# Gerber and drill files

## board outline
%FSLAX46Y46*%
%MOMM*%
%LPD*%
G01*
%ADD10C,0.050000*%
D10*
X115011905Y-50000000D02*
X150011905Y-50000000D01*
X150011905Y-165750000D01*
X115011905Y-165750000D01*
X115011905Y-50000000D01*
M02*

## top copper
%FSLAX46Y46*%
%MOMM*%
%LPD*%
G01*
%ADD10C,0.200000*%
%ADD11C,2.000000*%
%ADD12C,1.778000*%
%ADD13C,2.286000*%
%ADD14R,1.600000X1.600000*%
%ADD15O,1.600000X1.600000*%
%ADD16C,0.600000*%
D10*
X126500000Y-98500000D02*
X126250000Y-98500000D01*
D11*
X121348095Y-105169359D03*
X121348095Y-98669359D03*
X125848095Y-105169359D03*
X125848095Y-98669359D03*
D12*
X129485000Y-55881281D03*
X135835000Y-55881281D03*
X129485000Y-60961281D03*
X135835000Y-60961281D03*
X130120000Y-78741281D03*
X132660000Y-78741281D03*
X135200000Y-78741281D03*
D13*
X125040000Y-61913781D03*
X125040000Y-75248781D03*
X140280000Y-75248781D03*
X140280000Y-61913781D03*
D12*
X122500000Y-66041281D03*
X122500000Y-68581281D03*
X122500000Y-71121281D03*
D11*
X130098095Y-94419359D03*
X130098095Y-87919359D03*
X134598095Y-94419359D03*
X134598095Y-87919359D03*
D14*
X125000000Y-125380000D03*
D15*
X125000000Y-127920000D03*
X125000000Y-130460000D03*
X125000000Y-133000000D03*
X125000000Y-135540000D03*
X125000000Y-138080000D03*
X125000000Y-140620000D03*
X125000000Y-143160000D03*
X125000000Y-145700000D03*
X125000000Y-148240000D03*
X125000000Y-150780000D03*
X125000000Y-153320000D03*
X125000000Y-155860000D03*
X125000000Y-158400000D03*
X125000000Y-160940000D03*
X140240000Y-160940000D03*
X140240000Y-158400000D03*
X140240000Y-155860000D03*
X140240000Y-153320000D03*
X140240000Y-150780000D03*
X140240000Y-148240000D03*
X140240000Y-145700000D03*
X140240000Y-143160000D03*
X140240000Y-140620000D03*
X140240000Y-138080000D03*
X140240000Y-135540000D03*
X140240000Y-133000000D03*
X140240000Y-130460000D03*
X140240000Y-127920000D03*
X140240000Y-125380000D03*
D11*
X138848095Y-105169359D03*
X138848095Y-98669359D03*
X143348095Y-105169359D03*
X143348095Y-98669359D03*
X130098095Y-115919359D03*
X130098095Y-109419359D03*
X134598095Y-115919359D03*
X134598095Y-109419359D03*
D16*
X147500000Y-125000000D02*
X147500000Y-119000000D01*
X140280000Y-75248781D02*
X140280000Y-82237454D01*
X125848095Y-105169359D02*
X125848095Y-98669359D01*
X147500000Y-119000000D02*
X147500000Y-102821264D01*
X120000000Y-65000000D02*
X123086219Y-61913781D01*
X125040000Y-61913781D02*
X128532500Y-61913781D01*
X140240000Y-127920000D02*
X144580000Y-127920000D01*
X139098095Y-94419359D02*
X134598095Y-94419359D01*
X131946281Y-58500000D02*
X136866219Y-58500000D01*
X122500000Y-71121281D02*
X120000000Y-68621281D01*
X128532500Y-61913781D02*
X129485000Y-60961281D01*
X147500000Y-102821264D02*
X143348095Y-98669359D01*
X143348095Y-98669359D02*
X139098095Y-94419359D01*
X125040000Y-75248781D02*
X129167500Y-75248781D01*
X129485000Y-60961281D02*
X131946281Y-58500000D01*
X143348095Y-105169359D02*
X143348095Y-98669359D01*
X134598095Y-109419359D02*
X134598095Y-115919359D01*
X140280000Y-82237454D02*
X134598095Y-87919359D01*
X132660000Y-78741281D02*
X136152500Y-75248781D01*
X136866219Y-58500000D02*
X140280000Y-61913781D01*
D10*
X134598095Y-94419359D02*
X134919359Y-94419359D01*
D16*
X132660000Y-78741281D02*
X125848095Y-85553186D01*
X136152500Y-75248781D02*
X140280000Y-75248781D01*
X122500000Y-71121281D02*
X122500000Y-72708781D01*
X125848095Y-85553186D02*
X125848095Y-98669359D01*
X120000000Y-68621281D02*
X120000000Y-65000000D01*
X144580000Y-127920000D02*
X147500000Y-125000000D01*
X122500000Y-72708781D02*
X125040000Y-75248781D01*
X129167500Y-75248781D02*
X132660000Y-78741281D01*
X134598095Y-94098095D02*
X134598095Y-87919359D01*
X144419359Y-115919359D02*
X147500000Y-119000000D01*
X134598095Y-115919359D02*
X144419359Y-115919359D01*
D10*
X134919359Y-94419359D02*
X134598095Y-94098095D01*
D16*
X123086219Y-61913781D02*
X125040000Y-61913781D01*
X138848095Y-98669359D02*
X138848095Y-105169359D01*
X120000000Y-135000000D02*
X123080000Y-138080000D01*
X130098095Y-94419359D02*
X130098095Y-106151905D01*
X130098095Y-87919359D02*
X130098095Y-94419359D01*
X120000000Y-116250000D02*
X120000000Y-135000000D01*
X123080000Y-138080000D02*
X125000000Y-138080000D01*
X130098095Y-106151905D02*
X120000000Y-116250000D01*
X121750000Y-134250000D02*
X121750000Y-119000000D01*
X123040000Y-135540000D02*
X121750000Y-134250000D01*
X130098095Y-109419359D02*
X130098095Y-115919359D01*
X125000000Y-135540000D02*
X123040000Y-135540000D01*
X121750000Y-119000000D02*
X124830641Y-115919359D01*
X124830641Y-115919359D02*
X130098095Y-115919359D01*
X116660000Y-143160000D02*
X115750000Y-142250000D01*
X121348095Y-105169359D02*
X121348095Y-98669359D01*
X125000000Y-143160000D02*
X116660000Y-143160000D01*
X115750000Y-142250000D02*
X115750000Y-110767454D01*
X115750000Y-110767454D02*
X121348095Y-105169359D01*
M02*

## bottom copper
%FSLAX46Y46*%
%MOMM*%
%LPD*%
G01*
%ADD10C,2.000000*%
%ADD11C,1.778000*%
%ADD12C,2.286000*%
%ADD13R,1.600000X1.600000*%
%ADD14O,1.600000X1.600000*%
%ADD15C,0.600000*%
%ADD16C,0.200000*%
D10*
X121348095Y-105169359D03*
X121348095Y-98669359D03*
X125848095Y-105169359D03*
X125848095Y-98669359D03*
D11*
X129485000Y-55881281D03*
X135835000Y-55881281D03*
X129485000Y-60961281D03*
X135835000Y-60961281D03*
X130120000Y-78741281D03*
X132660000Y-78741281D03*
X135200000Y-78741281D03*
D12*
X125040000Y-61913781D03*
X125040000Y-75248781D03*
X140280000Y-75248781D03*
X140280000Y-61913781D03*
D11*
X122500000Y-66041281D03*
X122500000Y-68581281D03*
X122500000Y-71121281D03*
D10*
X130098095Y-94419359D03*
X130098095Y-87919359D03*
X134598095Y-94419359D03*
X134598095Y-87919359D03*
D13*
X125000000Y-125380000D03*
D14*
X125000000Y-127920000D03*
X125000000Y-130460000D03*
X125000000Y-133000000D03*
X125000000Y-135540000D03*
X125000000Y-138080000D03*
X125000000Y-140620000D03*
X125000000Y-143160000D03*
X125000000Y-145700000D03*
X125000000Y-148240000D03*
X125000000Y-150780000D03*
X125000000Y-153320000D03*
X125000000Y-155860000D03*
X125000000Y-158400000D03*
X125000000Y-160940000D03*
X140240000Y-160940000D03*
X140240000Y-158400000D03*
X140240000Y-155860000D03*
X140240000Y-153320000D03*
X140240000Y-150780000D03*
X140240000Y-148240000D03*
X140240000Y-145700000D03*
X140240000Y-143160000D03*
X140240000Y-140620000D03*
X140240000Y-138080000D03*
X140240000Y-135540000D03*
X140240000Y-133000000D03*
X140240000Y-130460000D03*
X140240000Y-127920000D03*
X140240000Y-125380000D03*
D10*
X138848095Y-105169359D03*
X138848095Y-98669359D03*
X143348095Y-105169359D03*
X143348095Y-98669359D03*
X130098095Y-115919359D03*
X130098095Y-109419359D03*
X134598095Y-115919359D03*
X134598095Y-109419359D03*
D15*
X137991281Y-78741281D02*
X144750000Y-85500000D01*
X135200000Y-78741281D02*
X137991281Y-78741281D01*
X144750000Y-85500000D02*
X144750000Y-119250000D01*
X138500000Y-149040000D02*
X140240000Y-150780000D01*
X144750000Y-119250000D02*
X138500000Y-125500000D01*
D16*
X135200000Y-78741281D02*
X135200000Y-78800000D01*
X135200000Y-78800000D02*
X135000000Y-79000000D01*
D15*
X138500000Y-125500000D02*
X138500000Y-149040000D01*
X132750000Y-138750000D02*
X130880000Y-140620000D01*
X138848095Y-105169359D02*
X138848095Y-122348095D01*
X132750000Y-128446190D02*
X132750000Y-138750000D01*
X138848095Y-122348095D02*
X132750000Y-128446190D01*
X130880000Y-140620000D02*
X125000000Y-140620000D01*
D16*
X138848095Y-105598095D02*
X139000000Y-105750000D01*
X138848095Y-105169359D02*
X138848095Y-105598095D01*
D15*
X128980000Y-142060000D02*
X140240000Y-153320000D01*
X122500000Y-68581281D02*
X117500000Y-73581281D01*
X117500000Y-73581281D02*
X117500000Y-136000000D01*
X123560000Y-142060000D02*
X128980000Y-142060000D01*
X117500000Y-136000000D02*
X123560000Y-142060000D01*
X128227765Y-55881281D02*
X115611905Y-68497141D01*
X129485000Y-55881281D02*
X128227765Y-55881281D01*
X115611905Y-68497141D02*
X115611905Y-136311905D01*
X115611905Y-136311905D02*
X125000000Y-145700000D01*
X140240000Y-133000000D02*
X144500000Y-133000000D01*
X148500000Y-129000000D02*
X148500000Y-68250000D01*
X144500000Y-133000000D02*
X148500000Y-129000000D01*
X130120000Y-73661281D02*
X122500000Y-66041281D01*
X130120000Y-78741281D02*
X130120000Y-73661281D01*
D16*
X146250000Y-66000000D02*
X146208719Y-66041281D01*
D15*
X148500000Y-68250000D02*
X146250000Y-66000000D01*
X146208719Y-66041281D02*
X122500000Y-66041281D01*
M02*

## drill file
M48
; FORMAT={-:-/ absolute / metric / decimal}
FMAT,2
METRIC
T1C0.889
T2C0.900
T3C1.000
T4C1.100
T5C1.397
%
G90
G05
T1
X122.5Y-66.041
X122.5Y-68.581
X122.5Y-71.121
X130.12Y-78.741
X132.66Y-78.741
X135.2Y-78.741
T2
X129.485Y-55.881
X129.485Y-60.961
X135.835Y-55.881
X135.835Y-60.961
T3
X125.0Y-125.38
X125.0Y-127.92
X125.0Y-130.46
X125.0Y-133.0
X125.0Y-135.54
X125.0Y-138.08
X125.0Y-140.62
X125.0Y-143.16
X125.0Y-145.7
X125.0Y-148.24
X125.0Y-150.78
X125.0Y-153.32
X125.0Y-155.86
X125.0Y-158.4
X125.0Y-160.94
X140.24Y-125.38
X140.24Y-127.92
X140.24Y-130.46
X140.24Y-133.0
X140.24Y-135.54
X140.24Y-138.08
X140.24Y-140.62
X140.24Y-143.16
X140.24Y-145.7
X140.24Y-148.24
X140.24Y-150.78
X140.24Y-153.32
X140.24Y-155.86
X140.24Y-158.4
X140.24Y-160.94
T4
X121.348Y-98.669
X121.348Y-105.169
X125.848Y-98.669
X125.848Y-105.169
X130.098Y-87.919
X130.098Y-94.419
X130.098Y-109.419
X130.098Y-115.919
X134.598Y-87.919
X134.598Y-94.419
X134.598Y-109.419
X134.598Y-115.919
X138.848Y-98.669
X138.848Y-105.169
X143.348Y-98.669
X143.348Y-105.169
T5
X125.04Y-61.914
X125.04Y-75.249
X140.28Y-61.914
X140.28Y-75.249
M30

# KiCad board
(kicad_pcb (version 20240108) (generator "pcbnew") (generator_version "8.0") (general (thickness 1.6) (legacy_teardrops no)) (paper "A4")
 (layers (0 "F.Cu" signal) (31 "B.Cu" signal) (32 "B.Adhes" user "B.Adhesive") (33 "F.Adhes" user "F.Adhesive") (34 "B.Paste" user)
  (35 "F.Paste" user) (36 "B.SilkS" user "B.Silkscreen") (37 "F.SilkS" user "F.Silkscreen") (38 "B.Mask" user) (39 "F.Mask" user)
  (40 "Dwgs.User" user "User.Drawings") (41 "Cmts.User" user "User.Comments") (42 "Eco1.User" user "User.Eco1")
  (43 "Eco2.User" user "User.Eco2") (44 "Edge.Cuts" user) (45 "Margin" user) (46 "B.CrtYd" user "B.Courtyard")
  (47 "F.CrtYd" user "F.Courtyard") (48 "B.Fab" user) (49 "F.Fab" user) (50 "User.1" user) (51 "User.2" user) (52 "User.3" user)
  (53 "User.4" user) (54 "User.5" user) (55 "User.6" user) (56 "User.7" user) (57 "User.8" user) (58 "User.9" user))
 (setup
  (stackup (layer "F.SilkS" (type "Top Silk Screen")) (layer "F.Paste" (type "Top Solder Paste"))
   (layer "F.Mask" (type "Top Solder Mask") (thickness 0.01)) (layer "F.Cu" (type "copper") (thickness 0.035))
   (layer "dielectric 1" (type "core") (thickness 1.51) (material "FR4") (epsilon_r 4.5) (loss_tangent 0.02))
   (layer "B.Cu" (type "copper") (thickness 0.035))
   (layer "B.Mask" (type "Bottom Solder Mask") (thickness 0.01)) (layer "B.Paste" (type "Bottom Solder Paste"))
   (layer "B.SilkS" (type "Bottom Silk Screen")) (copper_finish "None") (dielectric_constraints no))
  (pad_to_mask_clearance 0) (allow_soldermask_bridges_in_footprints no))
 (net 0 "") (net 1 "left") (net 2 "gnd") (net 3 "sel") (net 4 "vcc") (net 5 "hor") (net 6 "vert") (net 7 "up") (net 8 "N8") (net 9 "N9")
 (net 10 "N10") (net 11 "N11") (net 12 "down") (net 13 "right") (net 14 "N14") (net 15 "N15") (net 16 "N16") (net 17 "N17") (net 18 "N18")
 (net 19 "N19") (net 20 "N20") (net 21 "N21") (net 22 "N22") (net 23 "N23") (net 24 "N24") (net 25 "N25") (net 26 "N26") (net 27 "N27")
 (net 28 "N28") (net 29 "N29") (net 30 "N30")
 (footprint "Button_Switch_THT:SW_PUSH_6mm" (layer "F.Cu") (at 121.348095 105.169359 90)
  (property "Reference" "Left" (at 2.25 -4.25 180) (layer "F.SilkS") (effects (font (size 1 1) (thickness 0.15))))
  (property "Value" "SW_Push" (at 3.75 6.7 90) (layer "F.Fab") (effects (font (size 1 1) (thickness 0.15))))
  (pad "1" thru_hole circle (at 0 0 180) (size 2 2) (drill 1.1) (layers "*.Cu" "*.Mask") (remove_unused_layers no) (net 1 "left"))
  (pad "1" thru_hole circle (at 6.5 0 180) (size 2 2) (drill 1.1) (layers "*.Cu" "*.Mask") (remove_unused_layers no) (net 1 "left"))
  (pad "2" thru_hole circle (at 0 4.5 180) (size 2 2) (drill 1.1) (layers "*.Cu" "*.Mask") (remove_unused_layers no) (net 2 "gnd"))
  (pad "2" thru_hole circle (at 6.5 4.5 180) (size 2 2) (drill 1.1) (layers "*.Cu" "*.Mask") (remove_unused_layers no) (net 2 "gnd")))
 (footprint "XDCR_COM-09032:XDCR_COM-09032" (layer "F.Cu") (at 132.66 68.581281)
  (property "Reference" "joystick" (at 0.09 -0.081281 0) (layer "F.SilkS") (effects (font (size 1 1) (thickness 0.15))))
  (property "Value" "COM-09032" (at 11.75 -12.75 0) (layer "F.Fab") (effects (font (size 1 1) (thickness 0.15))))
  (pad "B1A" thru_hole circle (at -3.175 -12.7) (size 1.778 1.778) (drill 0.9) (layers "*.Cu" "*.Mask") (remove_unused_layers no)
   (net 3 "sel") (solder_mask_margin 0.102))
  (pad "B1B" thru_hole circle (at 3.175 -12.7) (size 1.778 1.778) (drill 0.9) (layers "*.Cu" "*.Mask") (remove_unused_layers no)
   (solder_mask_margin 0.102))
  (pad "B2A" thru_hole circle (at -3.175 -7.62) (size 1.778 1.778) (drill 0.9) (layers "*.Cu" "*.Mask") (remove_unused_layers no)
   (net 2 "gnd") (solder_mask_margin 0.102))
  (pad "B2B" thru_hole circle (at 3.175 -7.62) (size 1.778 1.778) (drill 0.9) (layers "*.Cu" "*.Mask") (remove_unused_layers no)
   (solder_mask_margin 0.102))
  (pad "H1" thru_hole circle (at -2.54 10.16) (size 1.778 1.778) (drill 0.889) (layers "*.Cu" "*.Mask") (remove_unused_layers no)
   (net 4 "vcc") (solder_mask_margin 0.102))
  (pad "H2" thru_hole circle (at 0 10.16) (size 1.778 1.778) (drill 0.889) (layers "*.Cu" "*.Mask") (remove_unused_layers no) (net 2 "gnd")
   (solder_mask_margin 0.102))
  (pad "H3" thru_hole circle (at 2.54 10.16) (size 1.778 1.778) (drill 0.889) (layers "*.Cu" "*.Mask") (remove_unused_layers no)
   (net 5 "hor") (solder_mask_margin 0.102))
  (pad "S1" thru_hole circle (at -7.62 -6.6675) (size 2.286 2.286) (drill 1.397) (layers "*.Cu" "*.Mask") (remove_unused_layers no)
   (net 2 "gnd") (solder_mask_margin 0.102))
  (pad "S2" thru_hole circle (at -7.62 6.6675) (size 2.286 2.286) (drill 1.397) (layers "*.Cu" "*.Mask") (remove_unused_layers no)
   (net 2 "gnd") (solder_mask_margin 0.102))
  (pad "S3" thru_hole circle (at 7.62 6.6675) (size 2.286 2.286) (drill 1.397) (layers "*.Cu" "*.Mask") (remove_unused_layers no)
   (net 2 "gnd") (solder_mask_margin 0.102))
  (pad "S4" thru_hole circle (at 7.62 -6.6675) (size 2.286 2.286) (drill 1.397) (layers "*.Cu" "*.Mask") (remove_unused_layers no)
   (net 2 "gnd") (solder_mask_margin 0.102))
  (pad "V1" thru_hole circle (at -10.16 -2.54) (size 1.778 1.778) (drill 0.889) (layers "*.Cu" "*.Mask") (remove_unused_layers no)
   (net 4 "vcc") (solder_mask_margin 0.102))
  (pad "V2" thru_hole circle (at -10.16 0) (size 1.778 1.778) (drill 0.889) (layers "*.Cu" "*.Mask") (remove_unused_layers no)
   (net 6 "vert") (solder_mask_margin 0.102))
  (pad "V3" thru_hole circle (at -10.16 2.54) (size 1.778 1.778) (drill 0.889) (layers "*.Cu" "*.Mask") (remove_unused_layers no)
   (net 2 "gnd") (solder_mask_margin 0.102)))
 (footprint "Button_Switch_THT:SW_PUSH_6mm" (layer "F.Cu") (at 130.098095 94.419359 90)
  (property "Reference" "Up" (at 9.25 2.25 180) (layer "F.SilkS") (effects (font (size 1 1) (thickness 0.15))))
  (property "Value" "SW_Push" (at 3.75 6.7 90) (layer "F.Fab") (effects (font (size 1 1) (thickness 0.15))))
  (pad "1" thru_hole circle (at 0 0 180) (size 2 2) (drill 1.1) (layers "*.Cu" "*.Mask") (remove_unused_layers no) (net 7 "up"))
  (pad "1" thru_hole circle (at 6.5 0 180) (size 2 2) (drill 1.1) (layers "*.Cu" "*.Mask") (remove_unused_layers no) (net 7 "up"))
  (pad "2" thru_hole circle (at 0 4.5 180) (size 2 2) (drill 1.1) (layers "*.Cu" "*.Mask") (remove_unused_layers no) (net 2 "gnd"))
  (pad "2" thru_hole circle (at 6.5 4.5 180) (size 2 2) (drill 1.1) (layers "*.Cu" "*.Mask") (remove_unused_layers no) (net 2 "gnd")))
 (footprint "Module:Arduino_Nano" (layer "F.Cu") (at 125 125.38)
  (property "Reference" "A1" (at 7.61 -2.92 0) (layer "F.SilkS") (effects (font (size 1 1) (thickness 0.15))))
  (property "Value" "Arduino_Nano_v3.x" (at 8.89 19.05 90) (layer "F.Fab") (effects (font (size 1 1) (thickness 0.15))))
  (pad "1" thru_hole rect (at 0 0) (size 1.6 1.6) (drill 1) (layers "*.Cu" "*.Mask") (remove_unused_layers no) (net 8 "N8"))
  (pad "2" thru_hole oval (at 0 2.54) (size 1.6 1.6) (drill 1) (layers "*.Cu" "*.Mask") (remove_unused_layers no) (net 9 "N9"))
  (pad "3" thru_hole oval (at 0 5.08) (size 1.6 1.6) (drill 1) (layers "*.Cu" "*.Mask") (remove_unused_layers no) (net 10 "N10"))
  (pad "4" thru_hole oval (at 0 7.62) (size 1.6 1.6) (drill 1) (layers "*.Cu" "*.Mask") (remove_unused_layers no) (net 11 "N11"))
  (pad "5" thru_hole oval (at 0 10.16) (size 1.6 1.6) (drill 1) (layers "*.Cu" "*.Mask") (remove_unused_layers no) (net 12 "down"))
  (pad "6" thru_hole oval (at 0 12.7) (size 1.6 1.6) (drill 1) (layers "*.Cu" "*.Mask") (remove_unused_layers no) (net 7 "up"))
  (pad "7" thru_hole oval (at 0 15.24) (size 1.6 1.6) (drill 1) (layers "*.Cu" "*.Mask") (remove_unused_layers no) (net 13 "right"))
  (pad "8" thru_hole oval (at 0 17.78) (size 1.6 1.6) (drill 1) (layers "*.Cu" "*.Mask") (remove_unused_layers no) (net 1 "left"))
  (pad "9" thru_hole oval (at 0 20.32) (size 1.6 1.6) (drill 1) (layers "*.Cu" "*.Mask") (remove_unused_layers no) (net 3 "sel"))
  (pad "10" thru_hole oval (at 0 22.86) (size 1.6 1.6) (drill 1) (layers "*.Cu" "*.Mask") (remove_unused_layers no) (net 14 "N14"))
  (pad "11" thru_hole oval (at 0 25.4) (size 1.6 1.6) (drill 1) (layers "*.Cu" "*.Mask") (remove_unused_layers no) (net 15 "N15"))
  (pad "12" thru_hole oval (at 0 27.94) (size 1.6 1.6) (drill 1) (layers "*.Cu" "*.Mask") (remove_unused_layers no) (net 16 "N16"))
  (pad "13" thru_hole oval (at 0 30.48) (size 1.6 1.6) (drill 1) (layers "*.Cu" "*.Mask") (remove_unused_layers no) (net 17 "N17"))
  (pad "14" thru_hole oval (at 0 33.02) (size 1.6 1.6) (drill 1) (layers "*.Cu" "*.Mask") (remove_unused_layers no) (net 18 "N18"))
  (pad "15" thru_hole oval (at 0 35.56) (size 1.6 1.6) (drill 1) (layers "*.Cu" "*.Mask") (remove_unused_layers no) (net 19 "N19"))
  (pad "16" thru_hole oval (at 15.24 35.56) (size 1.6 1.6) (drill 1) (layers "*.Cu" "*.Mask") (remove_unused_layers no) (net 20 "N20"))
  (pad "17" thru_hole oval (at 15.24 33.02) (size 1.6 1.6) (drill 1) (layers "*.Cu" "*.Mask") (remove_unused_layers no) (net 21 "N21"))
  (pad "18" thru_hole oval (at 15.24 30.48) (size 1.6 1.6) (drill 1) (layers "*.Cu" "*.Mask") (remove_unused_layers no) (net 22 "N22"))
  (pad "19" thru_hole oval (at 15.24 27.94) (size 1.6 1.6) (drill 1) (layers "*.Cu" "*.Mask") (remove_unused_layers no) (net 6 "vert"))
  (pad "20" thru_hole oval (at 15.24 25.4) (size 1.6 1.6) (drill 1) (layers "*.Cu" "*.Mask") (remove_unused_layers no) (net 5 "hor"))
  (pad "21" thru_hole oval (at 15.24 22.86) (size 1.6 1.6) (drill 1) (layers "*.Cu" "*.Mask") (remove_unused_layers no) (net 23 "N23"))
  (pad "22" thru_hole oval (at 15.24 20.32) (size 1.6 1.6) (drill 1) (layers "*.Cu" "*.Mask") (remove_unused_layers no) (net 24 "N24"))
  (pad "23" thru_hole oval (at 15.24 17.78) (size 1.6 1.6) (drill 1) (layers "*.Cu" "*.Mask") (remove_unused_layers no) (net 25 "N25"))
  (pad "24" thru_hole oval (at 15.24 15.24) (size 1.6 1.6) (drill 1) (layers "*.Cu" "*.Mask") (remove_unused_layers no) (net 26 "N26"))
  (pad "25" thru_hole oval (at 15.24 12.7) (size 1.6 1.6) (drill 1) (layers "*.Cu" "*.Mask") (remove_unused_layers no) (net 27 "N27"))
  (pad "26" thru_hole oval (at 15.24 10.16) (size 1.6 1.6) (drill 1) (layers "*.Cu" "*.Mask") (remove_unused_layers no) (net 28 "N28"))
  (pad "27" thru_hole oval (at 15.24 7.62) (size 1.6 1.6) (drill 1) (layers "*.Cu" "*.Mask") (remove_unused_layers no) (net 4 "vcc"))
  (pad "28" thru_hole oval (at 15.24 5.08) (size 1.6 1.6) (drill 1) (layers "*.Cu" "*.Mask") (remove_unused_layers no) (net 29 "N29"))
  (pad "29" thru_hole oval (at 15.24 2.54) (size 1.6 1.6) (drill 1) (layers "*.Cu" "*.Mask") (remove_unused_layers no) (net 2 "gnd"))
  (pad "30" thru_hole oval (at 15.24 0) (size 1.6 1.6) (drill 1) (layers "*.Cu" "*.Mask") (remove_unused_layers no) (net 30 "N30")))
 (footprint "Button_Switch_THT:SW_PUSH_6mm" (layer "F.Cu") (at 138.848095 105.169359 90)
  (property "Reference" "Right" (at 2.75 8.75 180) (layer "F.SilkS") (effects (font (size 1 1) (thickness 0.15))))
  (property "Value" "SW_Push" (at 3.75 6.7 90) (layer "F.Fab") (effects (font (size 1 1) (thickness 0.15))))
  (pad "1" thru_hole circle (at 0 0 180) (size 2 2) (drill 1.1) (layers "*.Cu" "*.Mask") (remove_unused_layers no) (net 13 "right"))
  (pad "1" thru_hole circle (at 6.5 0 180) (size 2 2) (drill 1.1) (layers "*.Cu" "*.Mask") (remove_unused_layers no) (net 13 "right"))
  (pad "2" thru_hole circle (at 0 4.5 180) (size 2 2) (drill 1.1) (layers "*.Cu" "*.Mask") (remove_unused_layers no) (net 2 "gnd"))
  (pad "2" thru_hole circle (at 6.5 4.5 180) (size 2 2) (drill 1.1) (layers "*.Cu" "*.Mask") (remove_unused_layers no) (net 2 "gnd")))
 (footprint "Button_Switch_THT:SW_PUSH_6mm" (layer "F.Cu") (at 130.098095 115.919359 90)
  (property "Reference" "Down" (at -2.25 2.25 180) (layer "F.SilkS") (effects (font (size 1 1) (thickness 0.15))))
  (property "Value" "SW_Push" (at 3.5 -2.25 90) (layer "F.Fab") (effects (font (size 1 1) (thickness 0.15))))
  (pad "1" thru_hole circle (at 0 0 180) (size 2 2) (drill 1.1) (layers "*.Cu" "*.Mask") (remove_unused_layers no) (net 12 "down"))
  (pad "1" thru_hole circle (at 6.5 0 180) (size 2 2) (drill 1.1) (layers "*.Cu" "*.Mask") (remove_unused_layers no) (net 12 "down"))
  (pad "2" thru_hole circle (at 0 4.5 180) (size 2 2) (drill 1.1) (layers "*.Cu" "*.Mask") (remove_unused_layers no) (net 2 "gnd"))
  (pad "2" thru_hole circle (at 6.5 4.5 180) (size 2 2) (drill 1.1) (layers "*.Cu" "*.Mask") (remove_unused_layers no) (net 2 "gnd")))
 (gr_line (start 126.5 98.5) (end 126.25 98.5) (stroke (width 0.2) (type default)) (layer "F.Cu") (net 2))
 (gr_rect (start 115.011905 50) (end 150.011905 165.75) (stroke (width 0.05) (type default)) (fill none) (layer "Edge.Cuts"))
 (segment (start 147.5 125) (end 147.5 119) (width 0.6) (layer "F.Cu") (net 2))
 (segment (start 140.28 75.248781) (end 140.28 82.237454) (width 0.6) (layer "F.Cu") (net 2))
 (segment (start 125.848095 105.169359) (end 125.848095 98.669359) (width 0.6) (layer "F.Cu") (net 2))
 (segment (start 147.5 119) (end 147.5 102.821264) (width 0.6) (layer "F.Cu") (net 2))
 (segment (start 120 65) (end 123.086219 61.913781) (width 0.6) (layer "F.Cu") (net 2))
 (segment (start 125.04 61.913781) (end 128.5325 61.913781) (width 0.6) (layer "F.Cu") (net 2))
 (segment (start 140.24 127.92) (end 144.58 127.92) (width 0.6) (layer "F.Cu") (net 2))
 (segment (start 139.098095 94.419359) (end 134.598095 94.419359) (width 0.6) (layer "F.Cu") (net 2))
 (segment (start 131.946281 58.5) (end 136.866219 58.5) (width 0.6) (layer "F.Cu") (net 2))
 (segment (start 122.5 71.121281) (end 120 68.621281) (width 0.6) (layer "F.Cu") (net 2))
 (segment (start 128.5325 61.913781) (end 129.485 60.961281) (width 0.6) (layer "F.Cu") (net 2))
 (segment (start 147.5 102.821264) (end 143.348095 98.669359) (width 0.6) (layer "F.Cu") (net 2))
 (segment (start 143.348095 98.669359) (end 139.098095 94.419359) (width 0.6) (layer "F.Cu") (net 2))
 (segment (start 125.04 75.248781) (end 129.1675 75.248781) (width 0.6) (layer "F.Cu") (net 2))
 (segment (start 129.485 60.961281) (end 131.946281 58.5) (width 0.6) (layer "F.Cu") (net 2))
 (segment (start 143.348095 105.169359) (end 143.348095 98.669359) (width 0.6) (layer "F.Cu") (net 2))
 (segment (start 134.598095 109.419359) (end 134.598095 115.919359) (width 0.6) (layer "F.Cu") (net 2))
 (segment (start 140.28 82.237454) (end 134.598095 87.919359) (width 0.6) (layer "F.Cu") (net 2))
 (segment (start 132.66 78.741281) (end 136.1525 75.248781) (width 0.6) (layer "F.Cu") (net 2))
 (segment (start 136.866219 58.5) (end 140.28 61.913781) (width 0.6) (layer "F.Cu") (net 2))
 (segment (start 134.598095 94.419359) (end 134.919359 94.419359) (width 0.2) (layer "F.Cu") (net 2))
 (segment (start 132.66 78.741281) (end 125.848095 85.553186) (width 0.6) (layer "F.Cu") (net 2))
 (segment (start 136.1525 75.248781) (end 140.28 75.248781) (width 0.6) (layer "F.Cu") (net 2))
 (segment (start 122.5 71.121281) (end 122.5 72.708781) (width 0.6) (layer "F.Cu") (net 2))
 (segment (start 125.848095 85.553186) (end 125.848095 98.669359) (width 0.6) (layer "F.Cu") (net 2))
 (segment (start 120 68.621281) (end 120 65) (width 0.6) (layer "F.Cu") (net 2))
 (segment (start 144.58 127.92) (end 147.5 125) (width 0.6) (layer "F.Cu") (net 2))
 (segment (start 122.5 72.708781) (end 125.04 75.248781) (width 0.6) (layer "F.Cu") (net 2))
 (segment (start 129.1675 75.248781) (end 132.66 78.741281) (width 0.6) (layer "F.Cu") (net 2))
 (segment (start 134.598095 94.098095) (end 134.598095 87.919359) (width 0.6) (layer "F.Cu") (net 2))
 (segment (start 144.419359 115.919359) (end 147.5 119) (width 0.6) (layer "F.Cu") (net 2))
 (segment (start 134.598095 115.919359) (end 144.419359 115.919359) (width 0.6) (layer "F.Cu") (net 2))
 (segment (start 134.919359 94.419359) (end 134.598095 94.098095) (width 0.2) (layer "F.Cu") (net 2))
 (segment (start 123.086219 61.913781) (end 125.04 61.913781) (width 0.6) (layer "F.Cu") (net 2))
 (segment (start 137.991281 78.741281) (end 144.75 85.5) (width 0.6) (layer "B.Cu") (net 5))
 (segment (start 135.2 78.741281) (end 137.991281 78.741281) (width 0.6) (layer "B.Cu") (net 5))
 (segment (start 144.75 85.5) (end 144.75 119.25) (width 0.6) (layer "B.Cu") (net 5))
 (segment (start 138.5 149.04) (end 140.24 150.78) (width 0.6) (layer "B.Cu") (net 5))
 (segment (start 144.75 119.25) (end 138.5 125.5) (width 0.6) (layer "B.Cu") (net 5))
 (segment (start 135.2 78.741281) (end 135.2 78.8) (width 0.2) (layer "B.Cu") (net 5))
 (segment (start 135.2 78.8) (end 135 79) (width 0.2) (layer "B.Cu") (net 5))
 (segment (start 138.5 125.5) (end 138.5 149.04) (width 0.6) (layer "B.Cu") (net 5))
 (segment (start 138.848095 98.669359) (end 138.848095 105.169359) (width 0.6) (layer "F.Cu") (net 13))
 (segment (start 132.75 138.75) (end 130.88 140.62) (width 0.6) (layer "B.Cu") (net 13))
 (segment (start 138.848095 105.169359) (end 138.848095 122.348095) (width 0.6) (layer "B.Cu") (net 13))
 (segment (start 132.75 128.44619) (end 132.75 138.75) (width 0.6) (layer "B.Cu") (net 13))
 (segment (start 138.848095 122.348095) (end 132.75 128.44619) (width 0.6) (layer "B.Cu") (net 13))
 (segment (start 130.88 140.62) (end 125 140.62) (width 0.6) (layer "B.Cu") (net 13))
 (segment (start 138.848095 105.598095) (end 139 105.75) (width 0.2) (layer "B.Cu") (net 13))
 (segment (start 138.848095 105.169359) (end 138.848095 105.598095) (width 0.2) (layer "B.Cu") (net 13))
 (segment (start 120 135) (end 123.08 138.08) (width 0.6) (layer "F.Cu") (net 7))
 (segment (start 130.098095 94.419359) (end 130.098095 106.151905) (width 0.6) (layer "F.Cu") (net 7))
 (segment (start 130.098095 87.919359) (end 130.098095 94.419359) (width 0.6) (layer "F.Cu") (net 7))
 (segment (start 120 116.25) (end 120 135) (width 0.6) (layer "F.Cu") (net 7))
 (segment (start 123.08 138.08) (end 125 138.08) (width 0.6) (layer "F.Cu") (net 7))
 (segment (start 130.098095 106.151905) (end 120 116.25) (width 0.6) (layer "F.Cu") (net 7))
 (segment (start 128.98 142.06) (end 140.24 153.32) (width 0.6) (layer "B.Cu") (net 6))
 (segment (start 122.5 68.581281) (end 117.5 73.581281) (width 0.6) (layer "B.Cu") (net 6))
 (segment (start 117.5 73.581281) (end 117.5 136) (width 0.6) (layer "B.Cu") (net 6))
 (segment (start 123.56 142.06) (end 128.98 142.06) (width 0.6) (layer "B.Cu") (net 6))
 (segment (start 117.5 136) (end 123.56 142.06) (width 0.6) (layer "B.Cu") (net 6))
 (segment (start 128.227765 55.881281) (end 115.611905 68.497141) (width 0.6) (layer "B.Cu") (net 3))
 (segment (start 129.485 55.881281) (end 128.227765 55.881281) (width 0.6) (layer "B.Cu") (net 3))
 (segment (start 115.611905 68.497141) (end 115.611905 136.311905) (width 0.6) (layer "B.Cu") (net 3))
 (segment (start 115.611905 136.311905) (end 125 145.7) (width 0.6) (layer "B.Cu") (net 3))
 (segment (start 140.24 133) (end 144.5 133) (width 0.6) (layer "B.Cu") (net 4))
 (segment (start 148.5 129) (end 148.5 68.25) (width 0.6) (layer "B.Cu") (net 4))
 (segment (start 144.5 133) (end 148.5 129) (width 0.6) (layer "B.Cu") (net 4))
 (segment (start 130.12 73.661281) (end 122.5 66.041281) (width 0.6) (layer "B.Cu") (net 4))
 (segment (start 130.12 78.741281) (end 130.12 73.661281) (width 0.6) (layer "B.Cu") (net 4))
 (segment (start 146.25 66) (end 146.208719 66.041281) (width 0.2) (layer "B.Cu") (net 4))
 (segment (start 148.5 68.25) (end 146.25 66) (width 0.6) (layer "B.Cu") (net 4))
 (segment (start 146.208719 66.041281) (end 122.5 66.041281) (width 0.6) (layer "B.Cu") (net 4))
 (segment (start 121.75 134.25) (end 121.75 119) (width 0.6) (layer "F.Cu") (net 12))
 (segment (start 123.04 135.54) (end 121.75 134.25) (width 0.6) (layer "F.Cu") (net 12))
 (segment (start 130.098095 109.419359) (end 130.098095 115.919359) (width 0.6) (layer "F.Cu") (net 12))
 (segment (start 125 135.54) (end 123.04 135.54) (width 0.6) (layer "F.Cu") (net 12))
 (segment (start 121.75 119) (end 124.830641 115.919359) (width 0.6) (layer "F.Cu") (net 12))
 (segment (start 124.830641 115.919359) (end 130.098095 115.919359) (width 0.6) (layer "F.Cu") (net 12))
 (segment (start 116.66 143.16) (end 115.75 142.25) (width 0.6) (layer "F.Cu") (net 1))
 (segment (start 121.348095 105.169359) (end 121.348095 98.669359) (width 0.6) (layer "F.Cu") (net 1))
 (segment (start 125 143.16) (end 116.66 143.16) (width 0.6) (layer "F.Cu") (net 1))
 (segment (start 115.75 142.25) (end 115.75 110.767454) (width 0.6) (layer "F.Cu") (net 1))
 (segment (start 115.75 110.767454) (end 121.348095 105.169359) (width 0.6) (layer "F.Cu") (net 1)))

